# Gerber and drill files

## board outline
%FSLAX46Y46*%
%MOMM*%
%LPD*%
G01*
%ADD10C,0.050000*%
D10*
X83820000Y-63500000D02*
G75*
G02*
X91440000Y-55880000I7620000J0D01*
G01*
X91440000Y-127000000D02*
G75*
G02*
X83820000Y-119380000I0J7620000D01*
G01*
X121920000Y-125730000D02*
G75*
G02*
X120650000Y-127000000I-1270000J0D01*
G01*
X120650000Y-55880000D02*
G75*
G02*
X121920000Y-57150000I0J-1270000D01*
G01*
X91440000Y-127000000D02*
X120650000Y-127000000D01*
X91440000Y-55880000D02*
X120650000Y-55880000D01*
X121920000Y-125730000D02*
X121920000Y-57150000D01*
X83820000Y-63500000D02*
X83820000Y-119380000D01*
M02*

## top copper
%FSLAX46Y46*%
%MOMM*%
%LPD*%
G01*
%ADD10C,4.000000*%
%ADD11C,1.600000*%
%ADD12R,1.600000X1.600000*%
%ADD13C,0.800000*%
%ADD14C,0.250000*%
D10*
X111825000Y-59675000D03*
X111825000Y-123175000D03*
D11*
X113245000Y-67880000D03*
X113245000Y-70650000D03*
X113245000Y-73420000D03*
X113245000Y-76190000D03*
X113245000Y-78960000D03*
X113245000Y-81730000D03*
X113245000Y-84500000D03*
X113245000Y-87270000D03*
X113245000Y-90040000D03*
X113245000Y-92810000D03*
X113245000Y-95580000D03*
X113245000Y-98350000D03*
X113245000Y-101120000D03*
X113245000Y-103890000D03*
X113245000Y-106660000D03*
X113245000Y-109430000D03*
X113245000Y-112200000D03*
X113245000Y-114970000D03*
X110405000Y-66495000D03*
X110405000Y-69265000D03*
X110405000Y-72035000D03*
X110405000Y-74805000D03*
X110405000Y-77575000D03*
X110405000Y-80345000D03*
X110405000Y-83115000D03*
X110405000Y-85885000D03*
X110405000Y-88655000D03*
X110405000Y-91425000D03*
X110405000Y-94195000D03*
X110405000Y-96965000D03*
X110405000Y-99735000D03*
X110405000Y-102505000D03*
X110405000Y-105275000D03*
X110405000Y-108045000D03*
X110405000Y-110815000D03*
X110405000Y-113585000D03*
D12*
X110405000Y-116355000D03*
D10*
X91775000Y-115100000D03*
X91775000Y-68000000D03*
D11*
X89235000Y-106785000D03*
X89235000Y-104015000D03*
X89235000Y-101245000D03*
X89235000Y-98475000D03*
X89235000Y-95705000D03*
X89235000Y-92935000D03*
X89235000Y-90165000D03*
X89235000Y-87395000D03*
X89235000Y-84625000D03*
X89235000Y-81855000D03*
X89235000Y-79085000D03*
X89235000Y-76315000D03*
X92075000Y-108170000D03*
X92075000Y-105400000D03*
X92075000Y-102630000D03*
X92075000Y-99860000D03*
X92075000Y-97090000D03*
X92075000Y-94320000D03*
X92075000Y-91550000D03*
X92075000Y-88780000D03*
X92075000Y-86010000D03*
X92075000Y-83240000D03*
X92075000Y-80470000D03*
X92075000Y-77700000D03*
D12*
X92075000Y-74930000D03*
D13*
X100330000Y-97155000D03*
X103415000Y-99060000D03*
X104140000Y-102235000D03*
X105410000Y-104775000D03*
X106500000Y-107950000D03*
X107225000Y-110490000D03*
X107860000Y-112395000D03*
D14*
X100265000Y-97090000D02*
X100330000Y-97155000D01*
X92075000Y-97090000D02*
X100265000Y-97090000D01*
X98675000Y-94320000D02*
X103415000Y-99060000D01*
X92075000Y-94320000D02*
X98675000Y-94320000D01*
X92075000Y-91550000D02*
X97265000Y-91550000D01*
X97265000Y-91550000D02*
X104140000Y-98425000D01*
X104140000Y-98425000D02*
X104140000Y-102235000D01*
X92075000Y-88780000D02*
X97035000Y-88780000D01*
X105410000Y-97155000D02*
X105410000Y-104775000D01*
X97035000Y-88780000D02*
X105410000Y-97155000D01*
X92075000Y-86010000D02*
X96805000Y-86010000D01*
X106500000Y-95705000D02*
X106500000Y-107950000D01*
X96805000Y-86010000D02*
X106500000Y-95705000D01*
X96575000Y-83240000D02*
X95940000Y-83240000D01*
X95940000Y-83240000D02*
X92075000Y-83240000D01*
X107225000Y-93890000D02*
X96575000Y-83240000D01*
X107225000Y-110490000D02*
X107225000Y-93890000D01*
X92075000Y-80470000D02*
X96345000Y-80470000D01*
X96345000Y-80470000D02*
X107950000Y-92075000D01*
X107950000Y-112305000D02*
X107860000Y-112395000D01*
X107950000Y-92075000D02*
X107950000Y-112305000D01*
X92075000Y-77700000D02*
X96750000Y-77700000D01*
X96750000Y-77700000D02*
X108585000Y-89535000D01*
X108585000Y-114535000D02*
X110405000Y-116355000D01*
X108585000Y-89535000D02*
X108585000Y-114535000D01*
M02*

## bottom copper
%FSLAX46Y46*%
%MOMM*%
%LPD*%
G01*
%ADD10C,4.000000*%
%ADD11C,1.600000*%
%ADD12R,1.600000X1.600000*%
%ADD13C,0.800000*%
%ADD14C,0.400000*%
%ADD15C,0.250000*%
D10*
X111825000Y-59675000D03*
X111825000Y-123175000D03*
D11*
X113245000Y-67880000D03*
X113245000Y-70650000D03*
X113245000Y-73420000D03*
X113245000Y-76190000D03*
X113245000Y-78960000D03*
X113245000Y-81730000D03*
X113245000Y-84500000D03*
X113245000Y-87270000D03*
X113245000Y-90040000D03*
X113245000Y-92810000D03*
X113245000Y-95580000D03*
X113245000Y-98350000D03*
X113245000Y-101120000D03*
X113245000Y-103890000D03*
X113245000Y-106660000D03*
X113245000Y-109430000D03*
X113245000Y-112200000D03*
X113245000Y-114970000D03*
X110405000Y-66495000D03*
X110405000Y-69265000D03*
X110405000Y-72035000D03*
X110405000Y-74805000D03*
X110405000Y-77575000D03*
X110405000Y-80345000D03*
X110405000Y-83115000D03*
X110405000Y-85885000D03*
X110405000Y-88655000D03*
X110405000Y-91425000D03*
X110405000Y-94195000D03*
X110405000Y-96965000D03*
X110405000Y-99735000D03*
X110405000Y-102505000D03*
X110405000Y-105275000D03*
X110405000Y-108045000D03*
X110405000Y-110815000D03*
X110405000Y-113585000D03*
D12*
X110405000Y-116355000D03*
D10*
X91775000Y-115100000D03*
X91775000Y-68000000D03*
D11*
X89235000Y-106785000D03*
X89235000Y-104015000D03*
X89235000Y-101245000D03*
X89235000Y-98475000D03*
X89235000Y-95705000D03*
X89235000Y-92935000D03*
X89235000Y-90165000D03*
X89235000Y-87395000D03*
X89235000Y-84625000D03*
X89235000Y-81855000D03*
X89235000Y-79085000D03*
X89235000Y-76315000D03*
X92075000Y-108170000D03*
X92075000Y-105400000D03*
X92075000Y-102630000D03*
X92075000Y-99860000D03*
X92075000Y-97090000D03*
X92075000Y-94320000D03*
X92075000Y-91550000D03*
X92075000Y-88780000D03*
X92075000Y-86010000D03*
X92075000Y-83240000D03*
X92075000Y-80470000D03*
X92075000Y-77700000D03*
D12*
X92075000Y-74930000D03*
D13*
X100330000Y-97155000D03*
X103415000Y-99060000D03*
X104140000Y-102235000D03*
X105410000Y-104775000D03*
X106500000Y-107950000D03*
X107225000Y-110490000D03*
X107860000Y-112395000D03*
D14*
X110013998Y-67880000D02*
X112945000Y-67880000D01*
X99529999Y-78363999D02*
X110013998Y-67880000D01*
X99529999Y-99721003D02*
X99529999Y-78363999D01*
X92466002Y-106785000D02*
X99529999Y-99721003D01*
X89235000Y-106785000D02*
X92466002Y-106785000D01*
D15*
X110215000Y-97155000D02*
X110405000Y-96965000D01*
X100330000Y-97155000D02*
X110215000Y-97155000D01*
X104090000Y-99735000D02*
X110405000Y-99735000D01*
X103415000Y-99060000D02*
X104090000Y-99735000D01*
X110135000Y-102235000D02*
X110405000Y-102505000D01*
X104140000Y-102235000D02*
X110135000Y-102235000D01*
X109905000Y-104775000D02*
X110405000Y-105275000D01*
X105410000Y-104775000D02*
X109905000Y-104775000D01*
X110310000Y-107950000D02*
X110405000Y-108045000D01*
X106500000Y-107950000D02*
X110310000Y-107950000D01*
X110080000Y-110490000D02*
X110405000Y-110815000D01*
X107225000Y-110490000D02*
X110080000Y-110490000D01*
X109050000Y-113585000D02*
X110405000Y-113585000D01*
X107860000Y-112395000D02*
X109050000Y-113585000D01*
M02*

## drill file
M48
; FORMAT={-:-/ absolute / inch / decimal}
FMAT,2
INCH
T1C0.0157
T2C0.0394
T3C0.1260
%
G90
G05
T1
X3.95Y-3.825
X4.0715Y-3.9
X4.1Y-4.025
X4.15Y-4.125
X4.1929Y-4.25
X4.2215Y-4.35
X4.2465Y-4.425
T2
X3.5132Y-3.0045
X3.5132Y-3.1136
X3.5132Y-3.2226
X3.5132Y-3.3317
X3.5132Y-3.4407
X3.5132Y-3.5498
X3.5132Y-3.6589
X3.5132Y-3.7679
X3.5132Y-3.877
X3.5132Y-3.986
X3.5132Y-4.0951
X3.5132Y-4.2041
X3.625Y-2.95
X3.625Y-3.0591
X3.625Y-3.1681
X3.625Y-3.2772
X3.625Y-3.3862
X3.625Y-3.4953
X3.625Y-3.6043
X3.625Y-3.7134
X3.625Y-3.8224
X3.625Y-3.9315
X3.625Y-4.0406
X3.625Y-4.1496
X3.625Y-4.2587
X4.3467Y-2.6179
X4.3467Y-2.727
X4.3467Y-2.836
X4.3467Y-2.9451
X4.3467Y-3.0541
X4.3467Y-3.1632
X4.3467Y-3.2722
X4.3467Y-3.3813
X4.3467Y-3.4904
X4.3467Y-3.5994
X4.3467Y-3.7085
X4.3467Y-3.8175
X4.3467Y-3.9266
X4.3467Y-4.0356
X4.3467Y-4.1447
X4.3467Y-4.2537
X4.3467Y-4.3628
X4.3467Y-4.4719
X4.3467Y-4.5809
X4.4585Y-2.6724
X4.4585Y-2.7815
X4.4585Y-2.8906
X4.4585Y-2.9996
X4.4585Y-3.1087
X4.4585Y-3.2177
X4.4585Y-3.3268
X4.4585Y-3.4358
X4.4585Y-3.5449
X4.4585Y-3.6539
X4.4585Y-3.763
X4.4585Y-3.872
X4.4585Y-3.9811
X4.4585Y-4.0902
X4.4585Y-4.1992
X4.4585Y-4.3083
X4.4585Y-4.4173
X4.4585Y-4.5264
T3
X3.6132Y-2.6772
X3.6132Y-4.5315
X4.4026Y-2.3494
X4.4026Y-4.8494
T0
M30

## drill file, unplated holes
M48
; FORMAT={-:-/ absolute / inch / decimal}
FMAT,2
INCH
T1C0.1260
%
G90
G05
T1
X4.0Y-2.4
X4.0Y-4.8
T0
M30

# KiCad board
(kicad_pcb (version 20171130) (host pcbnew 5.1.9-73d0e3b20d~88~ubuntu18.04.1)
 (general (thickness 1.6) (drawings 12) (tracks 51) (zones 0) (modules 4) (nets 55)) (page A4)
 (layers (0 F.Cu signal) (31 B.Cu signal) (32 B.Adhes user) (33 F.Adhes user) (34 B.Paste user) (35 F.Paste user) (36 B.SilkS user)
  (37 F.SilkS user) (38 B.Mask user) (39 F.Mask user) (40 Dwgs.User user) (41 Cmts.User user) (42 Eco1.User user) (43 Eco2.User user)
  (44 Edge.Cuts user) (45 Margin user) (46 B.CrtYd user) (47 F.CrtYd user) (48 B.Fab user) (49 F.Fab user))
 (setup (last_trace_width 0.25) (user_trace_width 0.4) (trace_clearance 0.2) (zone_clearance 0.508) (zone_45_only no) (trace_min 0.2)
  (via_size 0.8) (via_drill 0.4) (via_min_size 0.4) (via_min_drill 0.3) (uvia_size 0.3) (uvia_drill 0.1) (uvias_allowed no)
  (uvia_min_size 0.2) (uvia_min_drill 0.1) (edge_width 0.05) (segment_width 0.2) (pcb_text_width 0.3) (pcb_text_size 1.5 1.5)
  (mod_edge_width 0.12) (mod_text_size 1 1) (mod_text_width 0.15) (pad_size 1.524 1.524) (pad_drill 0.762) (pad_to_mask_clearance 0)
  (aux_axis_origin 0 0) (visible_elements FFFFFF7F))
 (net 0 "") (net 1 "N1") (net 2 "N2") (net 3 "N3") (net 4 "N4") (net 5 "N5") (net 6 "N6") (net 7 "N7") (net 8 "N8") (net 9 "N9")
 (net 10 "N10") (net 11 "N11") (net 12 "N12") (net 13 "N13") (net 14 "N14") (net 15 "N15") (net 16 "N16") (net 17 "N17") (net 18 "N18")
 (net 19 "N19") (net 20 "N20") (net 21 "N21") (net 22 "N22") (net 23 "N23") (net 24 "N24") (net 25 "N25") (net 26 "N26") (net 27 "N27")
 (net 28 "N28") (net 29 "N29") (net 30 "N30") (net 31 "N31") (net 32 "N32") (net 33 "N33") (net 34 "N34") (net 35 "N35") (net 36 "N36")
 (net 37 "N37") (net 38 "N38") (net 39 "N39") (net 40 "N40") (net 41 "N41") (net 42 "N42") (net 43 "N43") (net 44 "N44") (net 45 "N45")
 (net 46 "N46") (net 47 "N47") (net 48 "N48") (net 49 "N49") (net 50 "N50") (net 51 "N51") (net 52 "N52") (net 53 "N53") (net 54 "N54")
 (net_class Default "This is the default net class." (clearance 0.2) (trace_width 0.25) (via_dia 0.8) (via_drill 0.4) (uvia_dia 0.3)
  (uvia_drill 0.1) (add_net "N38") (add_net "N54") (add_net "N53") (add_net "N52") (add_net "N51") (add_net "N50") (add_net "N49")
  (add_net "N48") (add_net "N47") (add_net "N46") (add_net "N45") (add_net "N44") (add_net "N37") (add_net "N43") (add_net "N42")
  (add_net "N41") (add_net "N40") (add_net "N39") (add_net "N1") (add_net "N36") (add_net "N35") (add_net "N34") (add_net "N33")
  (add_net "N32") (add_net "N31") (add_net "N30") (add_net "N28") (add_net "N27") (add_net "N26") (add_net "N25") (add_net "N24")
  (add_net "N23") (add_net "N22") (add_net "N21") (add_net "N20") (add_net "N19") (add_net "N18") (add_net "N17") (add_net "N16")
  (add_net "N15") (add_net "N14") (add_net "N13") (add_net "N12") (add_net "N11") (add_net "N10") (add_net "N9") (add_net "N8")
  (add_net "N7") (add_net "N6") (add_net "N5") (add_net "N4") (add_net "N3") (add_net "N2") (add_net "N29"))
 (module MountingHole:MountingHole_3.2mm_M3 (layer F.Cu) (at 101.6 121.92)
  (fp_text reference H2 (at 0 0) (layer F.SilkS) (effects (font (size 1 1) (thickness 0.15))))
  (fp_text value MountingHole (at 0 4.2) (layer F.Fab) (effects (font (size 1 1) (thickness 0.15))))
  (pad 1 np_thru_hole circle (at 0 0) (size 3.2 3.2) (drill 3.2) (layers *.Cu *.Mask)))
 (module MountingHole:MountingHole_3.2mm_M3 (layer F.Cu) (at 101.6 60.96)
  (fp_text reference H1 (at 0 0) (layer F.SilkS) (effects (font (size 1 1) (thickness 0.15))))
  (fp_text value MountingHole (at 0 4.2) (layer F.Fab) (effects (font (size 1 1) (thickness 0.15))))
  (pad 1 np_thru_hole circle (at 0 0) (size 3.2 3.2) (drill 3.2) (layers *.Cu *.Mask)))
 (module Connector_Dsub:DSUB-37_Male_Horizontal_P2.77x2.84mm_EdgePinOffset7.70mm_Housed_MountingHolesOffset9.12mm (layer F.Cu)
  (at 110.405 116.355 90)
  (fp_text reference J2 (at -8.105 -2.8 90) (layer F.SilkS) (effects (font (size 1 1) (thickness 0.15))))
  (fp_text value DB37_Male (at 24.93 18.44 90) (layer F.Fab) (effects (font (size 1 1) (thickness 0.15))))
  (pad 0 thru_hole circle (at 56.68 1.42 90) (size 4 4) (drill 3.2) (layers *.Cu *.Mask))
  (pad 0 thru_hole circle (at -6.82 1.42 90) (size 4 4) (drill 3.2) (layers *.Cu *.Mask))
  (pad 37 thru_hole circle (at 48.475 2.84 90) (size 1.6 1.6) (drill 1) (layers *.Cu *.Mask) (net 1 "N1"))
  (pad 36 thru_hole circle (at 45.705 2.84 90) (size 1.6 1.6) (drill 1) (layers *.Cu *.Mask) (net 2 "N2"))
  (pad 35 thru_hole circle (at 42.935 2.84 90) (size 1.6 1.6) (drill 1) (layers *.Cu *.Mask) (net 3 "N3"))
  (pad 34 thru_hole circle (at 40.165 2.84 90) (size 1.6 1.6) (drill 1) (layers *.Cu *.Mask) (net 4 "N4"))
  (pad 33 thru_hole circle (at 37.395 2.84 90) (size 1.6 1.6) (drill 1) (layers *.Cu *.Mask) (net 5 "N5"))
  (pad 32 thru_hole circle (at 34.625 2.84 90) (size 1.6 1.6) (drill 1) (layers *.Cu *.Mask) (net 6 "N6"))
  (pad 31 thru_hole circle (at 31.855 2.84 90) (size 1.6 1.6) (drill 1) (layers *.Cu *.Mask) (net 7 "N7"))
  (pad 30 thru_hole circle (at 29.085 2.84 90) (size 1.6 1.6) (drill 1) (layers *.Cu *.Mask) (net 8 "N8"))
  (pad 29 thru_hole circle (at 26.315 2.84 90) (size 1.6 1.6) (drill 1) (layers *.Cu *.Mask) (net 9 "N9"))
  (pad 28 thru_hole circle (at 23.545 2.84 90) (size 1.6 1.6) (drill 1) (layers *.Cu *.Mask) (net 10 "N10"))
  (pad 27 thru_hole circle (at 20.775 2.84 90) (size 1.6 1.6) (drill 1) (layers *.Cu *.Mask) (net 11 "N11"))
  (pad 26 thru_hole circle (at 18.005 2.84 90) (size 1.6 1.6) (drill 1) (layers *.Cu *.Mask) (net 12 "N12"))
  (pad 25 thru_hole circle (at 15.235 2.84 90) (size 1.6 1.6) (drill 1) (layers *.Cu *.Mask) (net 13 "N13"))
  (pad 24 thru_hole circle (at 12.465 2.84 90) (size 1.6 1.6) (drill 1) (layers *.Cu *.Mask) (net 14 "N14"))
  (pad 23 thru_hole circle (at 9.695 2.84 90) (size 1.6 1.6) (drill 1) (layers *.Cu *.Mask) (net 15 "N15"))
  (pad 22 thru_hole circle (at 6.925 2.84 90) (size 1.6 1.6) (drill 1) (layers *.Cu *.Mask) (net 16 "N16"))
  (pad 21 thru_hole circle (at 4.155 2.84 90) (size 1.6 1.6) (drill 1) (layers *.Cu *.Mask) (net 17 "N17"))
  (pad 20 thru_hole circle (at 1.385 2.84 90) (size 1.6 1.6) (drill 1) (layers *.Cu *.Mask) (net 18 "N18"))
  (pad 19 thru_hole circle (at 49.86 0 90) (size 1.6 1.6) (drill 1) (layers *.Cu *.Mask) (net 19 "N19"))
  (pad 18 thru_hole circle (at 47.09 0 90) (size 1.6 1.6) (drill 1) (layers *.Cu *.Mask) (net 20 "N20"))
  (pad 17 thru_hole circle (at 44.32 0 90) (size 1.6 1.6) (drill 1) (layers *.Cu *.Mask) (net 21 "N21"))
  (pad 16 thru_hole circle (at 41.55 0 90) (size 1.6 1.6) (drill 1) (layers *.Cu *.Mask) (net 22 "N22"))
  (pad 15 thru_hole circle (at 38.78 0 90) (size 1.6 1.6) (drill 1) (layers *.Cu *.Mask) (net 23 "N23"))
  (pad 14 thru_hole circle (at 36.01 0 90) (size 1.6 1.6) (drill 1) (layers *.Cu *.Mask) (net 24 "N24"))
  (pad 13 thru_hole circle (at 33.24 0 90) (size 1.6 1.6) (drill 1) (layers *.Cu *.Mask) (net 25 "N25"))
  (pad 12 thru_hole circle (at 30.47 0 90) (size 1.6 1.6) (drill 1) (layers *.Cu *.Mask) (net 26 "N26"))
  (pad 11 thru_hole circle (at 27.7 0 90) (size 1.6 1.6) (drill 1) (layers *.Cu *.Mask) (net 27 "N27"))
  (pad 10 thru_hole circle (at 24.93 0 90) (size 1.6 1.6) (drill 1) (layers *.Cu *.Mask) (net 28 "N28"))
  (pad 9 thru_hole circle (at 22.16 0 90) (size 1.6 1.6) (drill 1) (layers *.Cu *.Mask) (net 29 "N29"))
  (pad 8 thru_hole circle (at 19.39 0 90) (size 1.6 1.6) (drill 1) (layers *.Cu *.Mask) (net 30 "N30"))
  (pad 7 thru_hole circle (at 16.62 0 90) (size 1.6 1.6) (drill 1) (layers *.Cu *.Mask) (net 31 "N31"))
  (pad 6 thru_hole circle (at 13.85 0 90) (size 1.6 1.6) (drill 1) (layers *.Cu *.Mask) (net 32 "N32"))
  (pad 5 thru_hole circle (at 11.08 0 90) (size 1.6 1.6) (drill 1) (layers *.Cu *.Mask) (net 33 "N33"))
  (pad 4 thru_hole circle (at 8.31 0 90) (size 1.6 1.6) (drill 1) (layers *.Cu *.Mask) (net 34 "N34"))
  (pad 3 thru_hole circle (at 5.54 0 90) (size 1.6 1.6) (drill 1) (layers *.Cu *.Mask) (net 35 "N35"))
  (pad 2 thru_hole circle (at 2.77 0 90) (size 1.6 1.6) (drill 1) (layers *.Cu *.Mask) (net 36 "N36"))
  (pad 1 thru_hole rect (at 0 0 90) (size 1.6 1.6) (drill 1) (layers *.Cu *.Mask) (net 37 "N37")))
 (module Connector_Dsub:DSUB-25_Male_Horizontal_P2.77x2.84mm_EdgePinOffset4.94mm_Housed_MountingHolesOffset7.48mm (layer F.Cu)
  (at 92.075 74.93 270)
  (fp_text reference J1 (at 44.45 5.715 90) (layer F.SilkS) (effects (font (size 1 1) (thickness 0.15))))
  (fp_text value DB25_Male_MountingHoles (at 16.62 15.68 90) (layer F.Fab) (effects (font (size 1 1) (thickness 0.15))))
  (pad 0 thru_hole circle (at 40.17 0.3 270) (size 4 4) (drill 3.2) (layers *.Cu *.Mask) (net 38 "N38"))
  (pad 0 thru_hole circle (at -6.93 0.3 270) (size 4 4) (drill 3.2) (layers *.Cu *.Mask) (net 38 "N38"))
  (pad 25 thru_hole circle (at 31.855 2.84 270) (size 1.6 1.6) (drill 1) (layers *.Cu *.Mask) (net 1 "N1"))
  (pad 24 thru_hole circle (at 29.085 2.84 270) (size 1.6 1.6) (drill 1) (layers *.Cu *.Mask) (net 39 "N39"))
  (pad 23 thru_hole circle (at 26.315 2.84 270) (size 1.6 1.6) (drill 1) (layers *.Cu *.Mask) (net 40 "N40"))
  (pad 22 thru_hole circle (at 23.545 2.84 270) (size 1.6 1.6) (drill 1) (layers *.Cu *.Mask) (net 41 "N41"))
  (pad 21 thru_hole circle (at 20.775 2.84 270) (size 1.6 1.6) (drill 1) (layers *.Cu *.Mask) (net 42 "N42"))
  (pad 20 thru_hole circle (at 18.005 2.84 270) (size 1.6 1.6) (drill 1) (layers *.Cu *.Mask) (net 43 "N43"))
  (pad 19 thru_hole circle (at 15.235 2.84 270) (size 1.6 1.6) (drill 1) (layers *.Cu *.Mask) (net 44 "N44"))
  (pad 18 thru_hole circle (at 12.465 2.84 270) (size 1.6 1.6) (drill 1) (layers *.Cu *.Mask) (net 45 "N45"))
  (pad 17 thru_hole circle (at 9.695 2.84 270) (size 1.6 1.6) (drill 1) (layers *.Cu *.Mask) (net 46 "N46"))
  (pad 16 thru_hole circle (at 6.925 2.84 270) (size 1.6 1.6) (drill 1) (layers *.Cu *.Mask) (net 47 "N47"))
  (pad 15 thru_hole circle (at 4.155 2.84 270) (size 1.6 1.6) (drill 1) (layers *.Cu *.Mask) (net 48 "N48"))
  (pad 14 thru_hole circle (at 1.385 2.84 270) (size 1.6 1.6) (drill 1) (layers *.Cu *.Mask) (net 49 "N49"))
  (pad 13 thru_hole circle (at 33.24 0 270) (size 1.6 1.6) (drill 1) (layers *.Cu *.Mask) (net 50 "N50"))
  (pad 12 thru_hole circle (at 30.47 0 270) (size 1.6 1.6) (drill 1) (layers *.Cu *.Mask) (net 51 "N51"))
  (pad 11 thru_hole circle (at 27.7 0 270) (size 1.6 1.6) (drill 1) (layers *.Cu *.Mask) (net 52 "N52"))
  (pad 10 thru_hole circle (at 24.93 0 270) (size 1.6 1.6) (drill 1) (layers *.Cu *.Mask) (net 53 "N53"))
  (pad 9 thru_hole circle (at 22.16 0 270) (size 1.6 1.6) (drill 1) (layers *.Cu *.Mask) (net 30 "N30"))
  (pad 8 thru_hole circle (at 19.39 0 270) (size 1.6 1.6) (drill 1) (layers *.Cu *.Mask) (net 31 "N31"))
  (pad 7 thru_hole circle (at 16.62 0 270) (size 1.6 1.6) (drill 1) (layers *.Cu *.Mask) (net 32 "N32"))
  (pad 6 thru_hole circle (at 13.85 0 270) (size 1.6 1.6) (drill 1) (layers *.Cu *.Mask) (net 33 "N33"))
  (pad 5 thru_hole circle (at 11.08 0 270) (size 1.6 1.6) (drill 1) (layers *.Cu *.Mask) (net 34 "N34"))
  (pad 4 thru_hole circle (at 8.31 0 270) (size 1.6 1.6) (drill 1) (layers *.Cu *.Mask) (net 35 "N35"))
  (pad 3 thru_hole circle (at 5.54 0 270) (size 1.6 1.6) (drill 1) (layers *.Cu *.Mask) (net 36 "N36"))
  (pad 2 thru_hole circle (at 2.77 0 270) (size 1.6 1.6) (drill 1) (layers *.Cu *.Mask) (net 37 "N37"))
  (pad 1 thru_hole rect (at 0 0 270) (size 1.6 1.6) (drill 1) (layers *.Cu *.Mask) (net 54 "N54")))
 (gr_arc (start 91.44 63.5) (end 91.44 55.88) (angle -90) (layer Edge.Cuts) (width 0.05))
 (gr_arc (start 91.44 119.38) (end 83.82 119.38) (angle -90) (layer Edge.Cuts) (width 0.05))
 (gr_arc (start 120.65 125.73) (end 120.65 127) (angle -90) (layer Edge.Cuts) (width 0.05))
 (gr_arc (start 120.65 57.15) (end 121.92 57.15) (angle -90) (layer Edge.Cuts) (width 0.05))
 (gr_line (start 91.44 127) (end 120.65 127) (layer Edge.Cuts) (width 0.05))
 (gr_line (start 91.44 55.88) (end 120.65 55.88) (layer Edge.Cuts) (width 0.05))
 (gr_line (start 121.92 125.73) (end 121.92 57.15) (layer Edge.Cuts) (width 0.05))
 (gr_line (start 83.82 63.5) (end 83.82 119.38) (layer Edge.Cuts) (width 0.05))
 (segment (start 110.013998 67.88) (end 112.945 67.88) (width 0.4) (layer B.Cu) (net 1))
 (segment (start 99.529999 78.363999) (end 110.013998 67.88) (width 0.4) (layer B.Cu) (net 1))
 (segment (start 99.529999 99.721003) (end 99.529999 78.363999) (width 0.4) (layer B.Cu) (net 1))
 (segment (start 92.466002 106.785) (end 99.529999 99.721003) (width 0.4) (layer B.Cu) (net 1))
 (segment (start 89.235 106.785) (end 92.466002 106.785) (width 0.4) (layer B.Cu) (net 1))
 (via (at 100.33 97.155) (size 0.8) (drill 0.4) (layers F.Cu B.Cu) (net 30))
 (segment (start 100.265 97.09) (end 100.33 97.155) (width 0.25) (layer F.Cu) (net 30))
 (segment (start 92.075 97.09) (end 100.265 97.09) (width 0.25) (layer F.Cu) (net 30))
 (segment (start 110.215 97.155) (end 110.405 96.965) (width 0.25) (layer B.Cu) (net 30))
 (segment (start 100.33 97.155) (end 110.215 97.155) (width 0.25) (layer B.Cu) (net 30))
 (via (at 103.415 99.06) (size 0.8) (drill 0.4) (layers F.Cu B.Cu) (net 31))
 (segment (start 98.675 94.32) (end 103.415 99.06) (width 0.25) (layer F.Cu) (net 31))
 (segment (start 92.075 94.32) (end 98.675 94.32) (width 0.25) (layer F.Cu) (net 31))
 (segment (start 104.09 99.735) (end 110.405 99.735) (width 0.25) (layer B.Cu) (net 31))
 (segment (start 103.415 99.06) (end 104.09 99.735) (width 0.25) (layer B.Cu) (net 31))
 (segment (start 92.075 91.55) (end 97.265 91.55) (width 0.25) (layer F.Cu) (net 32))
 (segment (start 97.265 91.55) (end 104.14 98.425) (width 0.25) (layer F.Cu) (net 32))
 (via (at 104.14 102.235) (size 0.8) (drill 0.4) (layers F.Cu B.Cu) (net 32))
 (segment (start 104.14 98.425) (end 104.14 102.235) (width 0.25) (layer F.Cu) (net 32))
 (segment (start 110.135 102.235) (end 110.405 102.505) (width 0.25) (layer B.Cu) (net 32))
 (segment (start 104.14 102.235) (end 110.135 102.235) (width 0.25) (layer B.Cu) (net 32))
 (segment (start 92.075 88.78) (end 97.035 88.78) (width 0.25) (layer F.Cu) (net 33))
 (via (at 105.41 104.775) (size 0.8) (drill 0.4) (layers F.Cu B.Cu) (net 33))
 (segment (start 105.41 97.155) (end 105.41 104.775) (width 0.25) (layer F.Cu) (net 33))
 (segment (start 97.035 88.78) (end 105.41 97.155) (width 0.25) (layer F.Cu) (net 33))
 (segment (start 109.905 104.775) (end 110.405 105.275) (width 0.25) (layer B.Cu) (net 33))
 (segment (start 105.41 104.775) (end 109.905 104.775) (width 0.25) (layer B.Cu) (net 33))
 (segment (start 92.075 86.01) (end 96.805 86.01) (width 0.25) (layer F.Cu) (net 34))
 (via (at 106.5 107.95) (size 0.8) (drill 0.4) (layers F.Cu B.Cu) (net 34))
 (segment (start 106.5 95.705) (end 106.5 107.95) (width 0.25) (layer F.Cu) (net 34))
 (segment (start 96.805 86.01) (end 106.5 95.705) (width 0.25) (layer F.Cu) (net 34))
 (segment (start 110.31 107.95) (end 110.405 108.045) (width 0.25) (layer B.Cu) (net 34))
 (segment (start 106.5 107.95) (end 110.31 107.95) (width 0.25) (layer B.Cu) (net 34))
 (via (at 107.225 110.49) (size 0.8) (drill 0.4) (layers F.Cu B.Cu) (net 35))
 (segment (start 110.08 110.49) (end 110.405 110.815) (width 0.25) (layer B.Cu) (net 35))
 (segment (start 107.225 110.49) (end 110.08 110.49) (width 0.25) (layer B.Cu) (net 35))
 (segment (start 96.575 83.24) (end 95.94 83.24) (width 0.25) (layer F.Cu) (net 35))
 (segment (start 95.94 83.24) (end 92.075 83.24) (width 0.25) (layer F.Cu) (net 35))
 (segment (start 107.225 93.89) (end 96.575 83.24) (width 0.25) (layer F.Cu) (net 35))
 (segment (start 107.225 110.49) (end 107.225 93.89) (width 0.25) (layer F.Cu) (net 35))
 (segment (start 92.075 80.47) (end 96.345 80.47) (width 0.25) (layer F.Cu) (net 36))
 (segment (start 96.345 80.47) (end 107.95 92.075) (width 0.25) (layer F.Cu) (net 36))
 (via (at 107.86 112.395) (size 0.8) (drill 0.4) (layers F.Cu B.Cu) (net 36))
 (segment (start 107.95 112.305) (end 107.86 112.395) (width 0.25) (layer F.Cu) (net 36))
 (segment (start 107.95 92.075) (end 107.95 112.305) (width 0.25) (layer F.Cu) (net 36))
 (segment (start 109.05 113.585) (end 110.405 113.585) (width 0.25) (layer B.Cu) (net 36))
 (segment (start 107.86 112.395) (end 109.05 113.585) (width 0.25) (layer B.Cu) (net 36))
 (segment (start 92.075 77.7) (end 96.75 77.7) (width 0.25) (layer F.Cu) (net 37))
 (segment (start 96.75 77.7) (end 108.585 89.535) (width 0.25) (layer F.Cu) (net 37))
 (segment (start 108.585 114.535) (end 110.405 116.355) (width 0.25) (layer F.Cu) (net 37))
 (segment (start 108.585 89.535) (end 108.585 114.535) (width 0.25) (layer F.Cu) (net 37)))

